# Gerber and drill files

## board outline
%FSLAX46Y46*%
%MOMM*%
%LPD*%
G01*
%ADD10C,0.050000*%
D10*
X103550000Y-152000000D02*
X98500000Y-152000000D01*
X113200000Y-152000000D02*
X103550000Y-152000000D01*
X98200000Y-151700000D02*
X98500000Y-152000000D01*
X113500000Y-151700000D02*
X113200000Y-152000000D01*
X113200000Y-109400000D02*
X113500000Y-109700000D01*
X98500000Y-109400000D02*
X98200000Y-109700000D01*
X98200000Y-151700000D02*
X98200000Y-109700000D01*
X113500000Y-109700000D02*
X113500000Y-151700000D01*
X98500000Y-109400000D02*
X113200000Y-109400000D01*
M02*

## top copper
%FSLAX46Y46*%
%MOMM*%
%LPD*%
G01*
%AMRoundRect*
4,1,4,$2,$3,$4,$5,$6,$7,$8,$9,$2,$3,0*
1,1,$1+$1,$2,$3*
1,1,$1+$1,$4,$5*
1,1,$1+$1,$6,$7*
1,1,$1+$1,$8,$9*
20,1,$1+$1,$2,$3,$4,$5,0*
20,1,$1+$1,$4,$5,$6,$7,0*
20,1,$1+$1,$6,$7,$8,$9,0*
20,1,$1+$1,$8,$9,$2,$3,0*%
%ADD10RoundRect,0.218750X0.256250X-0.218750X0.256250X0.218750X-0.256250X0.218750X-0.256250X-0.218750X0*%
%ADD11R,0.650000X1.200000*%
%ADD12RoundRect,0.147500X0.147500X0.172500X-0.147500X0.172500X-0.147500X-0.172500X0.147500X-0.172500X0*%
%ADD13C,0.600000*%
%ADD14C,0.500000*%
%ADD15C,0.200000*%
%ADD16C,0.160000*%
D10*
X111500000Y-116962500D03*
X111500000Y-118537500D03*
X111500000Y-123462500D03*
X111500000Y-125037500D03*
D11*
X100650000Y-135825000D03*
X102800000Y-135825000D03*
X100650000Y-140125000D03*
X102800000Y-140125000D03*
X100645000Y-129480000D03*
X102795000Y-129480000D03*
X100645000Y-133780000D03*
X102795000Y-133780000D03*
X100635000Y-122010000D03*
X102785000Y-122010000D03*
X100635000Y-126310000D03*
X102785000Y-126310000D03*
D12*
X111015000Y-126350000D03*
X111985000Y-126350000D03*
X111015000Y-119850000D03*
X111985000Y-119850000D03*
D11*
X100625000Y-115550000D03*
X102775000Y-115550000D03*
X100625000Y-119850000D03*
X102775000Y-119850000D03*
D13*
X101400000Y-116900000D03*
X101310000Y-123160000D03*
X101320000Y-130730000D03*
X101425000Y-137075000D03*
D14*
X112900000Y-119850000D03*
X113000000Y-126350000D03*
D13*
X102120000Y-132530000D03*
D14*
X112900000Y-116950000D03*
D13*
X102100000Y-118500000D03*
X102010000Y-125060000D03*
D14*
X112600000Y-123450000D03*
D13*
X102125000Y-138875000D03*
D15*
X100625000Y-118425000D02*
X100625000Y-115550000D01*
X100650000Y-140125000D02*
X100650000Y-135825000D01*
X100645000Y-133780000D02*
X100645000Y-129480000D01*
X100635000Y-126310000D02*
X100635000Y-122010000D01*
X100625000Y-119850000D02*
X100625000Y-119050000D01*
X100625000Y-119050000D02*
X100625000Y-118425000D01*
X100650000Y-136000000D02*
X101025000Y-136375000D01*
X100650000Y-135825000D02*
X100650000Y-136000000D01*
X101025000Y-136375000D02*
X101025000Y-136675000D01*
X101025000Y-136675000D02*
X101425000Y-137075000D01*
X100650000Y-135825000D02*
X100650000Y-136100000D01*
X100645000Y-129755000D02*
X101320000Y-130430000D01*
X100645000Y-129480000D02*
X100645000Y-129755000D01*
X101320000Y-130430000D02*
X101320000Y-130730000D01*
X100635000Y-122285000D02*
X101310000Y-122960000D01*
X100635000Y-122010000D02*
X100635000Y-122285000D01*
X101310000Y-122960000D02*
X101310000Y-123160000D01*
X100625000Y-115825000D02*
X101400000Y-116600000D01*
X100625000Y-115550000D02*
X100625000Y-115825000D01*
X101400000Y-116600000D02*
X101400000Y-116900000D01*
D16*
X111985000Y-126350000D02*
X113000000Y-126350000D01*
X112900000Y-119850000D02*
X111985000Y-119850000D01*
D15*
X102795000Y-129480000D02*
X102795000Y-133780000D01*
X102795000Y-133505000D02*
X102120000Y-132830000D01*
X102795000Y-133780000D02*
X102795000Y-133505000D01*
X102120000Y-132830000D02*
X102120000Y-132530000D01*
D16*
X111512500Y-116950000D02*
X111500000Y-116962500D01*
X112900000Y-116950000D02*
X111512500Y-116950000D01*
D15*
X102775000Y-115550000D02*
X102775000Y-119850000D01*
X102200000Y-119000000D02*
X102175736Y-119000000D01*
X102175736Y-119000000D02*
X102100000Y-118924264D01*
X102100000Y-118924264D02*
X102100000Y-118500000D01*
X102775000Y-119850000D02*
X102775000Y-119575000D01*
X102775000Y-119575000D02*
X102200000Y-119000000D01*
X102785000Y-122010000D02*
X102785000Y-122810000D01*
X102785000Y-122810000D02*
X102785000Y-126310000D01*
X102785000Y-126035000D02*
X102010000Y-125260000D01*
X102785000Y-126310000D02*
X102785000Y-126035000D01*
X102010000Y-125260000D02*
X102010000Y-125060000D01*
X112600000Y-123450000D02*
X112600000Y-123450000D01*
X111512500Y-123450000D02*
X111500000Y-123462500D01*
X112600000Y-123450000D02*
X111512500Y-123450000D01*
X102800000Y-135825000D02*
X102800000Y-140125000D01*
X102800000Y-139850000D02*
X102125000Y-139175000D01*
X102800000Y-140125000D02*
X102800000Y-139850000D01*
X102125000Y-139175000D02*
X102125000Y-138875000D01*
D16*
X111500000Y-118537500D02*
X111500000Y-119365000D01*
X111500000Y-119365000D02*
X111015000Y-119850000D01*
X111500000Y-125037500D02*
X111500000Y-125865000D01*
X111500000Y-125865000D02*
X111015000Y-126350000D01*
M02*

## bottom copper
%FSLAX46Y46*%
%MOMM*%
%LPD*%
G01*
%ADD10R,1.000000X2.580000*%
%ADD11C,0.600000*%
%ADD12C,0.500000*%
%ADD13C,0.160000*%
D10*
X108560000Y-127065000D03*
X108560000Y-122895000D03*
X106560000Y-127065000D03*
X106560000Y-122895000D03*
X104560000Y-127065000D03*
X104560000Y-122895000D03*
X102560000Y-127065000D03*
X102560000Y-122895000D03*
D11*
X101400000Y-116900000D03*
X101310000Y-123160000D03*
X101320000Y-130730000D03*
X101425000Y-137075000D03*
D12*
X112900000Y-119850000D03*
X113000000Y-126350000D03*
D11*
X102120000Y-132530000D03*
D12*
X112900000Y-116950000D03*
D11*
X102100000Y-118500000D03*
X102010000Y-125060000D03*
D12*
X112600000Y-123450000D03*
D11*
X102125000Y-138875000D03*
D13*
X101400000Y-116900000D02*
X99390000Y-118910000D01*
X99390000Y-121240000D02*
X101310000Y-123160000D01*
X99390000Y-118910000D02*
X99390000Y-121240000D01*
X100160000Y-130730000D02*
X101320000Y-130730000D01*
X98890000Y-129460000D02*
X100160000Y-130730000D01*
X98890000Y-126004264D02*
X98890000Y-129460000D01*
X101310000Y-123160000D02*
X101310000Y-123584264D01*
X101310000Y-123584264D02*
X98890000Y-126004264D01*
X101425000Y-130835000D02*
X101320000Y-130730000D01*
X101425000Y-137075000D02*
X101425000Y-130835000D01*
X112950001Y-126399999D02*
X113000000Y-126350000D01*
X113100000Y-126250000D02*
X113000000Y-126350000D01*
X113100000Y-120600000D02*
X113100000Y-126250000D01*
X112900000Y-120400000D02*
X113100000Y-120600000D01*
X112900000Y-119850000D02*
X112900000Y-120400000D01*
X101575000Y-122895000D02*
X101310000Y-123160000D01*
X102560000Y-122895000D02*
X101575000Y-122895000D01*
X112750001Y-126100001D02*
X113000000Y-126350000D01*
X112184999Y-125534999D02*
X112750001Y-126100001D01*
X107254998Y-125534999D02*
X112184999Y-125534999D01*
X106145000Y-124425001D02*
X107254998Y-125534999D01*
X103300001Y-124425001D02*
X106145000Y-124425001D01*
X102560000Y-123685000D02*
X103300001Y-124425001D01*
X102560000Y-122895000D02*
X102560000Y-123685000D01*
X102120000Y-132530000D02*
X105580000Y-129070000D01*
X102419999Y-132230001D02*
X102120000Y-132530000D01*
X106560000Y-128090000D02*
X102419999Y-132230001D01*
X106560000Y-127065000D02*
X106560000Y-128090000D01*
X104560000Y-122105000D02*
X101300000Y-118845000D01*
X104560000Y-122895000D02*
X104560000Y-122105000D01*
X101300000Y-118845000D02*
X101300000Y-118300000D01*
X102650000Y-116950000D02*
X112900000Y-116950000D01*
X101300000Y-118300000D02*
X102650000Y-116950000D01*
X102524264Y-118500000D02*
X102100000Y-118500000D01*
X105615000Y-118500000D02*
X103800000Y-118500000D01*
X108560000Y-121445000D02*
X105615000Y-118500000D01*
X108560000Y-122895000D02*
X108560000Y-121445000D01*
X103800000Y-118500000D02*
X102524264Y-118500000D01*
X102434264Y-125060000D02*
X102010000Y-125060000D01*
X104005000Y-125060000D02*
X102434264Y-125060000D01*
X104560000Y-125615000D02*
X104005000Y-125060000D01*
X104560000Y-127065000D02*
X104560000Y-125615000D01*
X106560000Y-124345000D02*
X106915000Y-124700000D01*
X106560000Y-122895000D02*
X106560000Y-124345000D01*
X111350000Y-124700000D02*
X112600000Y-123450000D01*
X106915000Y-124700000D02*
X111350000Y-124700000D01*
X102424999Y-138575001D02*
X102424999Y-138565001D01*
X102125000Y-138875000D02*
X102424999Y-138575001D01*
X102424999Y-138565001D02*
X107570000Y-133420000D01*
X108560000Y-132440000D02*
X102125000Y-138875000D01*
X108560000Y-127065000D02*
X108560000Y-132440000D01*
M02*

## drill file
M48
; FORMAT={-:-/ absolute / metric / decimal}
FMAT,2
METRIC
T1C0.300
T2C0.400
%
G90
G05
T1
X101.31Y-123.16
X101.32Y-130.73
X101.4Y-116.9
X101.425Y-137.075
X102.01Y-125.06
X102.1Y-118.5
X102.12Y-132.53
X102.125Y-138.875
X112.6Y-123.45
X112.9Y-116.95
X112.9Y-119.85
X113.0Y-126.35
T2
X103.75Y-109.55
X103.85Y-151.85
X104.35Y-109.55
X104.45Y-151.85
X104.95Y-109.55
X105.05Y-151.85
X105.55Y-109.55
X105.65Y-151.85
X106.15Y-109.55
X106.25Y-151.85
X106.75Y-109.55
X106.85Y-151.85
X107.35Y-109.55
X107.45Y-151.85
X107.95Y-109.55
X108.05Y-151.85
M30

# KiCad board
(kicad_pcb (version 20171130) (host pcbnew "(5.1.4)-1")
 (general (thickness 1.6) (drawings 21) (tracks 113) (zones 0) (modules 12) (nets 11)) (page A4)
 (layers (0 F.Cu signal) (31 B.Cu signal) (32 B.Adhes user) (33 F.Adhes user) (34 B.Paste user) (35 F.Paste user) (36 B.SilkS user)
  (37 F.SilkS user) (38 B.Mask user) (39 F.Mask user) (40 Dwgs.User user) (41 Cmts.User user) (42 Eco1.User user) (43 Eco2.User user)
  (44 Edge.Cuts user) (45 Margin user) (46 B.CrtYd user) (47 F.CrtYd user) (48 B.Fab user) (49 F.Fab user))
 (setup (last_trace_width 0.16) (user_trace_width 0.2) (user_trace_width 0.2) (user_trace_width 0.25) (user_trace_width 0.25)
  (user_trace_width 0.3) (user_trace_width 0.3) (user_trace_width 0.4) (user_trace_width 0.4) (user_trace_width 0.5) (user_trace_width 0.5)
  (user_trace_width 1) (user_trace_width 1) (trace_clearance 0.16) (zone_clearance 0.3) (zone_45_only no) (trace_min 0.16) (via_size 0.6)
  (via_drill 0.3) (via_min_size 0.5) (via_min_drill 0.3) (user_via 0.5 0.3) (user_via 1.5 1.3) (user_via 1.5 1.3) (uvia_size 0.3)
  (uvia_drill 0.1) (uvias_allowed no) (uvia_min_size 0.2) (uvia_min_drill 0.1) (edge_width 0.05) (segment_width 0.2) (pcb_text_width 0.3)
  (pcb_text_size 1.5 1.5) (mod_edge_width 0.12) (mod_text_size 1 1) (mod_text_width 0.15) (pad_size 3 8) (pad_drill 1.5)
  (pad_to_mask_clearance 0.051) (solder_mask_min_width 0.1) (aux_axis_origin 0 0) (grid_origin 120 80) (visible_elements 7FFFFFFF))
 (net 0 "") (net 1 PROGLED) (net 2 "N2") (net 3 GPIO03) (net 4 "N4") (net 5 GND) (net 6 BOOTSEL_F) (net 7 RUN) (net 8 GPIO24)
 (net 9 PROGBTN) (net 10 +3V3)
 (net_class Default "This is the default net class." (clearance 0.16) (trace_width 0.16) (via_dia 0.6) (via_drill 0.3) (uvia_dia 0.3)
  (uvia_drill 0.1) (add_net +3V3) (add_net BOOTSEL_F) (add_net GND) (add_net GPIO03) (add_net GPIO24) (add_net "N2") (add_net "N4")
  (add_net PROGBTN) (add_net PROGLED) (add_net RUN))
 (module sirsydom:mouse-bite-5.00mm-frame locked (layer F.Cu) (at 106.45 151.85 180)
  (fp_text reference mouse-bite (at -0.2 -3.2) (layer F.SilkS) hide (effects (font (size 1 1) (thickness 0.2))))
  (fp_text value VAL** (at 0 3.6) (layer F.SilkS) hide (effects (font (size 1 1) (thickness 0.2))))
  (pad "" np_thru_hole circle (at 1.4 0 180) (size 0.4 0.4) (drill 0.4) (layers *.Cu *.Mask))
  (pad "" np_thru_hole circle (at 0.8 0 180) (size 0.4 0.4) (drill 0.4) (layers *.Cu *.Mask))
  (pad "" np_thru_hole circle (at 2 0 180) (size 0.4 0.4) (drill 0.4) (layers *.Cu *.Mask))
  (pad "" np_thru_hole circle (at 2.6 0 180) (size 0.4 0.4) (drill 0.4) (layers *.Cu *.Mask))
  (pad "" np_thru_hole circle (at 0.2 0 180) (size 0.4 0.4) (drill 0.4) (layers *.Cu *.Mask))
  (pad "" np_thru_hole circle (at -1 0 180) (size 0.4 0.4) (drill 0.4) (layers *.Cu *.Mask))
  (pad "" np_thru_hole circle (at -1.6 0 180) (size 0.4 0.4) (drill 0.4) (layers *.Cu *.Mask))
  (pad "" np_thru_hole circle (at -0.4 0 180) (size 0.4 0.4) (drill 0.4) (layers *.Cu *.Mask)))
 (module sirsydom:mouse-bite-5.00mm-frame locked (layer F.Cu) (at 105.35 109.55)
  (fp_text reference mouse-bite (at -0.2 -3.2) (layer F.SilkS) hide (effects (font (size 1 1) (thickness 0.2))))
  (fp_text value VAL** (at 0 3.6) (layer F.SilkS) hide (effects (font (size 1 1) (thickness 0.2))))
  (pad "" np_thru_hole circle (at -0.4 0) (size 0.4 0.4) (drill 0.4) (layers *.Cu *.Mask))
  (pad "" np_thru_hole circle (at -1.6 0) (size 0.4 0.4) (drill 0.4) (layers *.Cu *.Mask))
  (pad "" np_thru_hole circle (at -1 0) (size 0.4 0.4) (drill 0.4) (layers *.Cu *.Mask))
  (pad "" np_thru_hole circle (at 0.2 0) (size 0.4 0.4) (drill 0.4) (layers *.Cu *.Mask))
  (pad "" np_thru_hole circle (at 2.6 0) (size 0.4 0.4) (drill 0.4) (layers *.Cu *.Mask))
  (pad "" np_thru_hole circle (at 2 0) (size 0.4 0.4) (drill 0.4) (layers *.Cu *.Mask))
  (pad "" np_thru_hole circle (at 0.8 0) (size 0.4 0.4) (drill 0.4) (layers *.Cu *.Mask))
  (pad "" np_thru_hole circle (at 1.4 0) (size 0.4 0.4) (drill 0.4) (layers *.Cu *.Mask)))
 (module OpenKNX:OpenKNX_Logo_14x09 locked (layer F.Cu) (at 105.8 146.4)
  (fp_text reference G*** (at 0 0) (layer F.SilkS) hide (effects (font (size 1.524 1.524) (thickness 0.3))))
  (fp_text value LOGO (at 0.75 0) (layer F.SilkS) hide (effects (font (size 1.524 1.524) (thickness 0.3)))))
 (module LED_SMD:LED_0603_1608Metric (layer F.Cu) (at 111.5 117.75 90)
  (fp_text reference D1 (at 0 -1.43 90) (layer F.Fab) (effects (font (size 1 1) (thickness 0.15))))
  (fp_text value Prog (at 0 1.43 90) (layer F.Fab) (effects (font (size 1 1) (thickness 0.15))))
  (pad 2 smd roundrect (at 0.7875 0 90) (size 0.875 0.95) (layers F.Cu F.Paste F.Mask) (roundrect_rratio 0.25) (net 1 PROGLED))
  (pad 1 smd roundrect (at -0.7875 0 90) (size 0.875 0.95) (layers F.Cu F.Paste F.Mask) (roundrect_rratio 0.25) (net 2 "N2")))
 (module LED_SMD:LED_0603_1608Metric (layer F.Cu) (at 111.5 124.25 90)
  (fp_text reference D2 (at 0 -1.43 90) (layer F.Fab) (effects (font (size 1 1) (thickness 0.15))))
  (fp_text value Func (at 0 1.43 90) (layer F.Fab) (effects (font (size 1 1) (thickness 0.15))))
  (pad 2 smd roundrect (at 0.7875 0 90) (size 0.875 0.95) (layers F.Cu F.Paste F.Mask) (roundrect_rratio 0.25) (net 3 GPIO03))
  (pad 1 smd roundrect (at -0.7875 0 90) (size 0.875 0.95) (layers F.Cu F.Paste F.Mask) (roundrect_rratio 0.25) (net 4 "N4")))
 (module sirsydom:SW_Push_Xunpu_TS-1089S (layer F.Cu) (at 101.725 137.975 270)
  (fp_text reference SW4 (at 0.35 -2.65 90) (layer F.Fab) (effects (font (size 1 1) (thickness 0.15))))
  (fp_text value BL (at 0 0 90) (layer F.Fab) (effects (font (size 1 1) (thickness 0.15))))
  (pad 2 smd rect (at -2.15 1.075 270) (size 1.2 0.65) (layers F.Cu F.Paste F.Mask) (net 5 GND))
  (pad 1 smd rect (at -2.15 -1.075 270) (size 1.2 0.65) (layers F.Cu F.Paste F.Mask) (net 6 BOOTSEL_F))
  (pad 2 smd rect (at 2.15 1.075 270) (size 1.2 0.65) (layers F.Cu F.Paste F.Mask) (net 5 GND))
  (pad 1 smd rect (at 2.15 -1.075 270) (size 1.2 0.65) (layers F.Cu F.Paste F.Mask) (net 6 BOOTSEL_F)))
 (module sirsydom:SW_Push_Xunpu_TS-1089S (layer F.Cu) (at 101.72 131.63 270)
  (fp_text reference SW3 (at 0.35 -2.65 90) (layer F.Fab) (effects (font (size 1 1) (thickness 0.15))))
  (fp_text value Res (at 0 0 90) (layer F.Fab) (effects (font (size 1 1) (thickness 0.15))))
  (pad 2 smd rect (at -2.15 1.075 270) (size 1.2 0.65) (layers F.Cu F.Paste F.Mask) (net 5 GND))
  (pad 1 smd rect (at -2.15 -1.075 270) (size 1.2 0.65) (layers F.Cu F.Paste F.Mask) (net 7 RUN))
  (pad 2 smd rect (at 2.15 1.075 270) (size 1.2 0.65) (layers F.Cu F.Paste F.Mask) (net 5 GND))
  (pad 1 smd rect (at 2.15 -1.075 270) (size 1.2 0.65) (layers F.Cu F.Paste F.Mask) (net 7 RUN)))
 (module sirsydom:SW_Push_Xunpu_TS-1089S (layer F.Cu) (at 101.71 124.16 270)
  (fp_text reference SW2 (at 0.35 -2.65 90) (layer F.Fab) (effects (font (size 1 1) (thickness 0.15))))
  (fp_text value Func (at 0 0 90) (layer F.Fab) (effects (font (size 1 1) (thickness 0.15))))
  (pad 2 smd rect (at -2.15 1.075 270) (size 1.2 0.65) (layers F.Cu F.Paste F.Mask) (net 5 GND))
  (pad 1 smd rect (at -2.15 -1.075 270) (size 1.2 0.65) (layers F.Cu F.Paste F.Mask) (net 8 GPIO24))
  (pad 2 smd rect (at 2.15 1.075 270) (size 1.2 0.65) (layers F.Cu F.Paste F.Mask) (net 5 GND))
  (pad 1 smd rect (at 2.15 -1.075 270) (size 1.2 0.65) (layers F.Cu F.Paste F.Mask) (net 8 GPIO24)))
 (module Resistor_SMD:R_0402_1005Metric (layer F.Cu) (at 111.5 126.35 180)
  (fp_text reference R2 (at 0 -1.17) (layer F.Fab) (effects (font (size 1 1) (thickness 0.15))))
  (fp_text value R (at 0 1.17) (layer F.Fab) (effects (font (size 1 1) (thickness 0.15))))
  (pad 2 smd roundrect (at 0.485 0 180) (size 0.59 0.64) (layers F.Cu F.Paste F.Mask) (roundrect_rratio 0.25) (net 4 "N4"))
  (pad 1 smd roundrect (at -0.485 0 180) (size 0.59 0.64) (layers F.Cu F.Paste F.Mask) (roundrect_rratio 0.25) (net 5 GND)))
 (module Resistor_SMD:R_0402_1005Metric (layer F.Cu) (at 111.5 119.85 180)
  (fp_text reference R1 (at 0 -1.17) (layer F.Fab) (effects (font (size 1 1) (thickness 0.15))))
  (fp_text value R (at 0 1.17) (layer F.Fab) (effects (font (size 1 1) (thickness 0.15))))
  (pad 2 smd roundrect (at 0.485 0 180) (size 0.59 0.64) (layers F.Cu F.Paste F.Mask) (roundrect_rratio 0.25) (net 2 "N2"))
  (pad 1 smd roundrect (at -0.485 0 180) (size 0.59 0.64) (layers F.Cu F.Paste F.Mask) (roundrect_rratio 0.25) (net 5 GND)))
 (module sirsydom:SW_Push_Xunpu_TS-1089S (layer F.Cu) (at 101.7 117.7 270)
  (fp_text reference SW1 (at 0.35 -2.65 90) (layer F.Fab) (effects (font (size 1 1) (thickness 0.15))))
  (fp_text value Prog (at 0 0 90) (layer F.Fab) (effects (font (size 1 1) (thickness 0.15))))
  (pad 2 smd rect (at -2.15 1.075 270) (size 1.2 0.65) (layers F.Cu F.Paste F.Mask) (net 5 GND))
  (pad 1 smd rect (at -2.15 -1.075 270) (size 1.2 0.65) (layers F.Cu F.Paste F.Mask) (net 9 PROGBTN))
  (pad 2 smd rect (at 2.15 1.075 270) (size 1.2 0.65) (layers F.Cu F.Paste F.Mask) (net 5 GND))
  (pad 1 smd rect (at 2.15 -1.075 270) (size 1.2 0.65) (layers F.Cu F.Paste F.Mask) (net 9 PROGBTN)))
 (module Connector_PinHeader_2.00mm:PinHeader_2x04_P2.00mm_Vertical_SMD (layer B.Cu) (at 105.56 124.98 270)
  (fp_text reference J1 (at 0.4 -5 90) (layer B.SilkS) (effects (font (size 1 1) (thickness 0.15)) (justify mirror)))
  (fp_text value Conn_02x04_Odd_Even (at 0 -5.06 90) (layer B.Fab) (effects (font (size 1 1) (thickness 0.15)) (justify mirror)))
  (pad 8 smd rect (at 2.085 -3 270) (size 2.58 1) (layers B.Cu B.Paste B.Mask) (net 6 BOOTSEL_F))
  (pad 7 smd rect (at -2.085 -3 270) (size 2.58 1) (layers B.Cu B.Paste B.Mask) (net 9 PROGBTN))
  (pad 6 smd rect (at 2.085 -1 270) (size 2.58 1) (layers B.Cu B.Paste B.Mask) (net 7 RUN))
  (pad 5 smd rect (at -2.085 -1 270) (size 2.58 1) (layers B.Cu B.Paste B.Mask) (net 3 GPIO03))
  (pad 4 smd rect (at 2.085 1 270) (size 2.58 1) (layers B.Cu B.Paste B.Mask) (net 8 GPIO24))
  (pad 3 smd rect (at -2.085 1 270) (size 2.58 1) (layers B.Cu B.Paste B.Mask) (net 1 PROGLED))
  (pad 2 smd rect (at 2.085 3 270) (size 2.58 1) (layers B.Cu B.Paste B.Mask) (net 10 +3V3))
  (pad 1 smd rect (at -2.085 3 270) (size 2.58 1) (layers B.Cu B.Paste B.Mask) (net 5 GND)))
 (gr_line (start 103.55 152) (end 98.5 152) (layer Edge.Cuts) (width 0.05))
 (gr_line (start 113.2 152) (end 103.55 152) (layer Edge.Cuts) (width 0.05))
 (gr_line (start 98.2 151.7) (end 98.5 152) (layer Edge.Cuts) (width 0.05))
 (gr_line (start 113.5 151.7) (end 113.2 152) (layer Edge.Cuts) (width 0.05))
 (gr_line (start 113.2 109.4) (end 113.5 109.7) (layer Edge.Cuts) (width 0.05))
 (gr_line (start 98.5 109.4) (end 98.2 109.7) (layer Edge.Cuts) (width 0.05))
 (gr_line (start 98.2 151.7) (end 98.2 109.7) (layer Edge.Cuts) (width 0.05))
 (gr_line (start 113.5 109.7) (end 113.5 151.7) (layer Edge.Cuts) (width 0.05))
 (gr_line (start 98.5 109.4) (end 113.2 109.4) (layer Edge.Cuts) (width 0.05))
 (segment (start 100.625 118.425) (end 100.625 115.55) (width 0.2) (layer F.Cu) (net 5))
 (segment (start 100.65 140.125) (end 100.65 135.825) (width 0.2) (layer F.Cu) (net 5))
 (segment (start 100.645 133.78) (end 100.645 129.48) (width 0.2) (layer F.Cu) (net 5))
 (segment (start 100.635 126.31) (end 100.635 122.01) (width 0.2) (layer F.Cu) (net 5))
 (segment (start 100.625 119.85) (end 100.625 119.05) (width 0.2) (layer F.Cu) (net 5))
 (segment (start 100.625 119.05) (end 100.625 118.425) (width 0.2) (layer F.Cu) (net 5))
 (segment (start 100.65 136) (end 101.025 136.375) (width 0.2) (layer F.Cu) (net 5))
 (segment (start 100.65 135.825) (end 100.65 136) (width 0.2) (layer F.Cu) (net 5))
 (segment (start 101.025 136.375) (end 101.025 136.675) (width 0.2) (layer F.Cu) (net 5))
 (segment (start 101.025 136.675) (end 101.425 137.075) (width 0.2) (layer F.Cu) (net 5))
 (segment (start 100.65 135.825) (end 100.65 136.1) (width 0.2) (layer F.Cu) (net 5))
 (segment (start 100.645 129.755) (end 101.32 130.43) (width 0.2) (layer F.Cu) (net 5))
 (segment (start 100.645 129.48) (end 100.645 129.755) (width 0.2) (layer F.Cu) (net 5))
 (segment (start 101.32 130.43) (end 101.32 130.73) (width 0.2) (layer F.Cu) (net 5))
 (segment (start 100.635 122.285) (end 101.31 122.96) (width 0.2) (layer F.Cu) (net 5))
 (segment (start 100.635 122.01) (end 100.635 122.285) (width 0.2) (layer F.Cu) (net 5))
 (segment (start 101.31 122.96) (end 101.31 123.16) (width 0.2) (layer F.Cu) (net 5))
 (segment (start 100.625 115.825) (end 101.4 116.6) (width 0.2) (layer F.Cu) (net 5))
 (segment (start 100.625 115.55) (end 100.625 115.825) (width 0.2) (layer F.Cu) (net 5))
 (segment (start 101.4 116.6) (end 101.4 116.9) (width 0.2) (layer F.Cu) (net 5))
 (via (at 101.4 116.9) (size 0.6) (drill 0.3) (layers F.Cu B.Cu) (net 5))
 (via (at 101.31 123.16) (size 0.6) (drill 0.3) (layers F.Cu B.Cu) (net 5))
 (via (at 101.32 130.73) (size 0.6) (drill 0.3) (layers F.Cu B.Cu) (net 5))
 (via (at 101.425 137.075) (size 0.6) (drill 0.3) (layers F.Cu B.Cu) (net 5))
 (via (at 112.9 119.85) (size 0.5) (drill 0.3) (layers F.Cu B.Cu) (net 5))
 (via (at 113 126.35) (size 0.5) (drill 0.3) (layers F.Cu B.Cu) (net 5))
 (segment (start 101.4 116.9) (end 99.39 118.91) (width 0.16) (layer B.Cu) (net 5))
 (segment (start 99.39 121.24) (end 101.31 123.16) (width 0.16) (layer B.Cu) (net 5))
 (segment (start 99.39 118.91) (end 99.39 121.24) (width 0.16) (layer B.Cu) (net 5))
 (segment (start 100.16 130.73) (end 101.32 130.73) (width 0.16) (layer B.Cu) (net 5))
 (segment (start 98.89 129.46) (end 100.16 130.73) (width 0.16) (layer B.Cu) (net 5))
 (segment (start 98.89 126.004264) (end 98.89 129.46) (width 0.16) (layer B.Cu) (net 5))
 (segment (start 101.31 123.16) (end 101.31 123.584264) (width 0.16) (layer B.Cu) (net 5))
 (segment (start 101.31 123.584264) (end 98.89 126.004264) (width 0.16) (layer B.Cu) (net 5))
 (segment (start 101.425 130.835) (end 101.32 130.73) (width 0.16) (layer B.Cu) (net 5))
 (segment (start 101.425 137.075) (end 101.425 130.835) (width 0.16) (layer B.Cu) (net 5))
 (segment (start 111.985 126.35) (end 113 126.35) (width 0.16) (layer F.Cu) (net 5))
 (segment (start 112.9 119.85) (end 111.985 119.85) (width 0.16) (layer F.Cu) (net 5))
 (segment (start 112.950001 126.399999) (end 113 126.35) (width 0.16) (layer B.Cu) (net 5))
 (segment (start 113.1 126.25) (end 113 126.35) (width 0.16) (layer B.Cu) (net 5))
 (segment (start 113.1 120.6) (end 113.1 126.25) (width 0.16) (layer B.Cu) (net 5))
 (segment (start 112.9 120.4) (end 113.1 120.6) (width 0.16) (layer B.Cu) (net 5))
 (segment (start 112.9 119.85) (end 112.9 120.4) (width 0.16) (layer B.Cu) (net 5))
 (segment (start 101.575 122.895) (end 101.31 123.16) (width 0.16) (layer B.Cu) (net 5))
 (segment (start 102.56 122.895) (end 101.575 122.895) (width 0.16) (layer B.Cu) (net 5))
 (segment (start 112.750001 126.100001) (end 113 126.35) (width 0.16) (layer B.Cu) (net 5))
 (segment (start 112.184999 125.534999) (end 112.750001 126.100001) (width 0.16) (layer B.Cu) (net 5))
 (segment (start 107.254998 125.534999) (end 112.184999 125.534999) (width 0.16) (layer B.Cu) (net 5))
 (segment (start 106.145 124.425001) (end 107.254998 125.534999) (width 0.16) (layer B.Cu) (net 5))
 (segment (start 103.300001 124.425001) (end 106.145 124.425001) (width 0.16) (layer B.Cu) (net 5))
 (segment (start 102.56 123.685) (end 103.300001 124.425001) (width 0.16) (layer B.Cu) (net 5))
 (segment (start 102.56 122.895) (end 102.56 123.685) (width 0.16) (layer B.Cu) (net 5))
 (segment (start 102.795 129.48) (end 102.795 133.78) (width 0.2) (layer F.Cu) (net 7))
 (segment (start 102.795 133.505) (end 102.12 132.83) (width 0.2) (layer F.Cu) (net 7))
 (segment (start 102.795 133.78) (end 102.795 133.505) (width 0.2) (layer F.Cu) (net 7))
 (segment (start 102.12 132.83) (end 102.12 132.53) (width 0.2) (layer F.Cu) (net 7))
 (via (at 102.12 132.53) (size 0.6) (drill 0.3) (layers F.Cu B.Cu) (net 7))
 (segment (start 102.12 132.53) (end 105.58 129.07) (width 0.16) (layer B.Cu) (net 7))
 (segment (start 102.419999 132.230001) (end 102.12 132.53) (width 0.16) (layer B.Cu) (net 7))
 (segment (start 106.56 128.09) (end 102.419999 132.230001) (width 0.16) (layer B.Cu) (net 7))
 (segment (start 106.56 127.065) (end 106.56 128.09) (width 0.16) (layer B.Cu) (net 7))
 (via (at 112.9 116.95) (size 0.5) (drill 0.3) (layers F.Cu B.Cu) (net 1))
 (segment (start 111.5125 116.95) (end 111.5 116.9625) (width 0.16) (layer F.Cu) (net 1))
 (segment (start 112.9 116.95) (end 111.5125 116.95) (width 0.16) (layer F.Cu) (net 1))
 (segment (start 104.56 122.105) (end 101.3 118.845) (width 0.16) (layer B.Cu) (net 1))
 (segment (start 104.56 122.895) (end 104.56 122.105) (width 0.16) (layer B.Cu) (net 1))
 (segment (start 101.3 118.845) (end 101.3 118.3) (width 0.16) (layer B.Cu) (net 1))
 (segment (start 102.65 116.95) (end 112.9 116.95) (width 0.16) (layer B.Cu) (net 1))
 (segment (start 101.3 118.3) (end 102.65 116.95) (width 0.16) (layer B.Cu) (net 1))
 (segment (start 102.775 115.55) (end 102.775 119.85) (width 0.2) (layer F.Cu) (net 9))
 (segment (start 102.2 119) (end 102.175736 119) (width 0.2) (layer F.Cu) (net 9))
 (segment (start 102.175736 119) (end 102.1 118.924264) (width 0.2) (layer F.Cu) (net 9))
 (segment (start 102.1 118.924264) (end 102.1 118.5) (width 0.2) (layer F.Cu) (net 9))
 (segment (start 102.775 119.85) (end 102.775 119.575) (width 0.2) (layer F.Cu) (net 9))
 (segment (start 102.775 119.575) (end 102.2 119) (width 0.2) (layer F.Cu) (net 9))
 (via (at 102.1 118.5) (size 0.6) (drill 0.3) (layers F.Cu B.Cu) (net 9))
 (segment (start 102.524264 118.5) (end 102.1 118.5) (width 0.16) (layer B.Cu) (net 9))
 (segment (start 105.615 118.5) (end 103.8 118.5) (width 0.16) (layer B.Cu) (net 9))
 (segment (start 108.56 121.445) (end 105.615 118.5) (width 0.16) (layer B.Cu) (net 9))
 (segment (start 108.56 122.895) (end 108.56 121.445) (width 0.16) (layer B.Cu) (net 9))
 (segment (start 103.8 118.5) (end 102.524264 118.5) (width 0.16) (layer B.Cu) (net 9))
 (segment (start 102.785 122.01) (end 102.785 122.81) (width 0.2) (layer F.Cu) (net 8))
 (segment (start 102.785 122.81) (end 102.785 126.31) (width 0.2) (layer F.Cu) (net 8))
 (segment (start 102.785 126.035) (end 102.01 125.26) (width 0.2) (layer F.Cu) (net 8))
 (segment (start 102.785 126.31) (end 102.785 126.035) (width 0.2) (layer F.Cu) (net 8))
 (segment (start 102.01 125.26) (end 102.01 125.06) (width 0.2) (layer F.Cu) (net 8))
 (via (at 102.01 125.06) (size 0.6) (drill 0.3) (layers F.Cu B.Cu) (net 8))
 (segment (start 102.434264 125.06) (end 102.01 125.06) (width 0.16) (layer B.Cu) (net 8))
 (segment (start 104.005 125.06) (end 102.434264 125.06) (width 0.16) (layer B.Cu) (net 8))
 (segment (start 104.56 125.615) (end 104.005 125.06) (width 0.16) (layer B.Cu) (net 8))
 (segment (start 104.56 127.065) (end 104.56 125.615) (width 0.16) (layer B.Cu) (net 8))
 (segment (start 112.6 123.45) (end 112.6 123.45) (width 0.2) (layer F.Cu) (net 3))
 (segment (start 111.5125 123.45) (end 111.5 123.4625) (width 0.2) (layer F.Cu) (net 3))
 (segment (start 112.6 123.45) (end 111.5125 123.45) (width 0.2) (layer F.Cu) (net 3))
 (via (at 112.6 123.45) (size 0.5) (drill 0.3) (layers F.Cu B.Cu) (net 3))
 (segment (start 106.56 124.345) (end 106.915 124.7) (width 0.16) (layer B.Cu) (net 3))
 (segment (start 106.56 122.895) (end 106.56 124.345) (width 0.16) (layer B.Cu) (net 3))
 (segment (start 111.35 124.7) (end 112.6 123.45) (width 0.16) (layer B.Cu) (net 3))
 (segment (start 106.915 124.7) (end 111.35 124.7) (width 0.16) (layer B.Cu) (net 3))
 (segment (start 102.8 135.825) (end 102.8 140.125) (width 0.2) (layer F.Cu) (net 6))
 (segment (start 102.8 139.85) (end 102.125 139.175) (width 0.2) (layer F.Cu) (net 6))
 (segment (start 102.8 140.125) (end 102.8 139.85) (width 0.2) (layer F.Cu) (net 6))
 (segment (start 102.125 139.175) (end 102.125 138.875) (width 0.2) (layer F.Cu) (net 6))
 (via (at 102.125 138.875) (size 0.6) (drill 0.3) (layers F.Cu B.Cu) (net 6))
 (segment (start 102.424999 138.575001) (end 102.424999 138.565001) (width 0.16) (layer B.Cu) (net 6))
 (segment (start 102.125 138.875) (end 102.424999 138.575001) (width 0.16) (layer B.Cu) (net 6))
 (segment (start 102.424999 138.565001) (end 107.57 133.42) (width 0.16) (layer B.Cu) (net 6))
 (segment (start 108.56 132.44) (end 102.125 138.875) (width 0.16) (layer B.Cu) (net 6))
 (segment (start 108.56 127.065) (end 108.56 132.44) (width 0.16) (layer B.Cu) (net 6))
 (segment (start 111.5 118.5375) (end 111.5 119.365) (width 0.16) (layer F.Cu) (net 2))
 (segment (start 111.5 119.365) (end 111.015 119.85) (width 0.16) (layer F.Cu) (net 2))
 (segment (start 111.5 125.0375) (end 111.5 125.865) (width 0.16) (layer F.Cu) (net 4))
 (segment (start 111.5 125.865) (end 111.015 126.35) (width 0.16) (layer F.Cu) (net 4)))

